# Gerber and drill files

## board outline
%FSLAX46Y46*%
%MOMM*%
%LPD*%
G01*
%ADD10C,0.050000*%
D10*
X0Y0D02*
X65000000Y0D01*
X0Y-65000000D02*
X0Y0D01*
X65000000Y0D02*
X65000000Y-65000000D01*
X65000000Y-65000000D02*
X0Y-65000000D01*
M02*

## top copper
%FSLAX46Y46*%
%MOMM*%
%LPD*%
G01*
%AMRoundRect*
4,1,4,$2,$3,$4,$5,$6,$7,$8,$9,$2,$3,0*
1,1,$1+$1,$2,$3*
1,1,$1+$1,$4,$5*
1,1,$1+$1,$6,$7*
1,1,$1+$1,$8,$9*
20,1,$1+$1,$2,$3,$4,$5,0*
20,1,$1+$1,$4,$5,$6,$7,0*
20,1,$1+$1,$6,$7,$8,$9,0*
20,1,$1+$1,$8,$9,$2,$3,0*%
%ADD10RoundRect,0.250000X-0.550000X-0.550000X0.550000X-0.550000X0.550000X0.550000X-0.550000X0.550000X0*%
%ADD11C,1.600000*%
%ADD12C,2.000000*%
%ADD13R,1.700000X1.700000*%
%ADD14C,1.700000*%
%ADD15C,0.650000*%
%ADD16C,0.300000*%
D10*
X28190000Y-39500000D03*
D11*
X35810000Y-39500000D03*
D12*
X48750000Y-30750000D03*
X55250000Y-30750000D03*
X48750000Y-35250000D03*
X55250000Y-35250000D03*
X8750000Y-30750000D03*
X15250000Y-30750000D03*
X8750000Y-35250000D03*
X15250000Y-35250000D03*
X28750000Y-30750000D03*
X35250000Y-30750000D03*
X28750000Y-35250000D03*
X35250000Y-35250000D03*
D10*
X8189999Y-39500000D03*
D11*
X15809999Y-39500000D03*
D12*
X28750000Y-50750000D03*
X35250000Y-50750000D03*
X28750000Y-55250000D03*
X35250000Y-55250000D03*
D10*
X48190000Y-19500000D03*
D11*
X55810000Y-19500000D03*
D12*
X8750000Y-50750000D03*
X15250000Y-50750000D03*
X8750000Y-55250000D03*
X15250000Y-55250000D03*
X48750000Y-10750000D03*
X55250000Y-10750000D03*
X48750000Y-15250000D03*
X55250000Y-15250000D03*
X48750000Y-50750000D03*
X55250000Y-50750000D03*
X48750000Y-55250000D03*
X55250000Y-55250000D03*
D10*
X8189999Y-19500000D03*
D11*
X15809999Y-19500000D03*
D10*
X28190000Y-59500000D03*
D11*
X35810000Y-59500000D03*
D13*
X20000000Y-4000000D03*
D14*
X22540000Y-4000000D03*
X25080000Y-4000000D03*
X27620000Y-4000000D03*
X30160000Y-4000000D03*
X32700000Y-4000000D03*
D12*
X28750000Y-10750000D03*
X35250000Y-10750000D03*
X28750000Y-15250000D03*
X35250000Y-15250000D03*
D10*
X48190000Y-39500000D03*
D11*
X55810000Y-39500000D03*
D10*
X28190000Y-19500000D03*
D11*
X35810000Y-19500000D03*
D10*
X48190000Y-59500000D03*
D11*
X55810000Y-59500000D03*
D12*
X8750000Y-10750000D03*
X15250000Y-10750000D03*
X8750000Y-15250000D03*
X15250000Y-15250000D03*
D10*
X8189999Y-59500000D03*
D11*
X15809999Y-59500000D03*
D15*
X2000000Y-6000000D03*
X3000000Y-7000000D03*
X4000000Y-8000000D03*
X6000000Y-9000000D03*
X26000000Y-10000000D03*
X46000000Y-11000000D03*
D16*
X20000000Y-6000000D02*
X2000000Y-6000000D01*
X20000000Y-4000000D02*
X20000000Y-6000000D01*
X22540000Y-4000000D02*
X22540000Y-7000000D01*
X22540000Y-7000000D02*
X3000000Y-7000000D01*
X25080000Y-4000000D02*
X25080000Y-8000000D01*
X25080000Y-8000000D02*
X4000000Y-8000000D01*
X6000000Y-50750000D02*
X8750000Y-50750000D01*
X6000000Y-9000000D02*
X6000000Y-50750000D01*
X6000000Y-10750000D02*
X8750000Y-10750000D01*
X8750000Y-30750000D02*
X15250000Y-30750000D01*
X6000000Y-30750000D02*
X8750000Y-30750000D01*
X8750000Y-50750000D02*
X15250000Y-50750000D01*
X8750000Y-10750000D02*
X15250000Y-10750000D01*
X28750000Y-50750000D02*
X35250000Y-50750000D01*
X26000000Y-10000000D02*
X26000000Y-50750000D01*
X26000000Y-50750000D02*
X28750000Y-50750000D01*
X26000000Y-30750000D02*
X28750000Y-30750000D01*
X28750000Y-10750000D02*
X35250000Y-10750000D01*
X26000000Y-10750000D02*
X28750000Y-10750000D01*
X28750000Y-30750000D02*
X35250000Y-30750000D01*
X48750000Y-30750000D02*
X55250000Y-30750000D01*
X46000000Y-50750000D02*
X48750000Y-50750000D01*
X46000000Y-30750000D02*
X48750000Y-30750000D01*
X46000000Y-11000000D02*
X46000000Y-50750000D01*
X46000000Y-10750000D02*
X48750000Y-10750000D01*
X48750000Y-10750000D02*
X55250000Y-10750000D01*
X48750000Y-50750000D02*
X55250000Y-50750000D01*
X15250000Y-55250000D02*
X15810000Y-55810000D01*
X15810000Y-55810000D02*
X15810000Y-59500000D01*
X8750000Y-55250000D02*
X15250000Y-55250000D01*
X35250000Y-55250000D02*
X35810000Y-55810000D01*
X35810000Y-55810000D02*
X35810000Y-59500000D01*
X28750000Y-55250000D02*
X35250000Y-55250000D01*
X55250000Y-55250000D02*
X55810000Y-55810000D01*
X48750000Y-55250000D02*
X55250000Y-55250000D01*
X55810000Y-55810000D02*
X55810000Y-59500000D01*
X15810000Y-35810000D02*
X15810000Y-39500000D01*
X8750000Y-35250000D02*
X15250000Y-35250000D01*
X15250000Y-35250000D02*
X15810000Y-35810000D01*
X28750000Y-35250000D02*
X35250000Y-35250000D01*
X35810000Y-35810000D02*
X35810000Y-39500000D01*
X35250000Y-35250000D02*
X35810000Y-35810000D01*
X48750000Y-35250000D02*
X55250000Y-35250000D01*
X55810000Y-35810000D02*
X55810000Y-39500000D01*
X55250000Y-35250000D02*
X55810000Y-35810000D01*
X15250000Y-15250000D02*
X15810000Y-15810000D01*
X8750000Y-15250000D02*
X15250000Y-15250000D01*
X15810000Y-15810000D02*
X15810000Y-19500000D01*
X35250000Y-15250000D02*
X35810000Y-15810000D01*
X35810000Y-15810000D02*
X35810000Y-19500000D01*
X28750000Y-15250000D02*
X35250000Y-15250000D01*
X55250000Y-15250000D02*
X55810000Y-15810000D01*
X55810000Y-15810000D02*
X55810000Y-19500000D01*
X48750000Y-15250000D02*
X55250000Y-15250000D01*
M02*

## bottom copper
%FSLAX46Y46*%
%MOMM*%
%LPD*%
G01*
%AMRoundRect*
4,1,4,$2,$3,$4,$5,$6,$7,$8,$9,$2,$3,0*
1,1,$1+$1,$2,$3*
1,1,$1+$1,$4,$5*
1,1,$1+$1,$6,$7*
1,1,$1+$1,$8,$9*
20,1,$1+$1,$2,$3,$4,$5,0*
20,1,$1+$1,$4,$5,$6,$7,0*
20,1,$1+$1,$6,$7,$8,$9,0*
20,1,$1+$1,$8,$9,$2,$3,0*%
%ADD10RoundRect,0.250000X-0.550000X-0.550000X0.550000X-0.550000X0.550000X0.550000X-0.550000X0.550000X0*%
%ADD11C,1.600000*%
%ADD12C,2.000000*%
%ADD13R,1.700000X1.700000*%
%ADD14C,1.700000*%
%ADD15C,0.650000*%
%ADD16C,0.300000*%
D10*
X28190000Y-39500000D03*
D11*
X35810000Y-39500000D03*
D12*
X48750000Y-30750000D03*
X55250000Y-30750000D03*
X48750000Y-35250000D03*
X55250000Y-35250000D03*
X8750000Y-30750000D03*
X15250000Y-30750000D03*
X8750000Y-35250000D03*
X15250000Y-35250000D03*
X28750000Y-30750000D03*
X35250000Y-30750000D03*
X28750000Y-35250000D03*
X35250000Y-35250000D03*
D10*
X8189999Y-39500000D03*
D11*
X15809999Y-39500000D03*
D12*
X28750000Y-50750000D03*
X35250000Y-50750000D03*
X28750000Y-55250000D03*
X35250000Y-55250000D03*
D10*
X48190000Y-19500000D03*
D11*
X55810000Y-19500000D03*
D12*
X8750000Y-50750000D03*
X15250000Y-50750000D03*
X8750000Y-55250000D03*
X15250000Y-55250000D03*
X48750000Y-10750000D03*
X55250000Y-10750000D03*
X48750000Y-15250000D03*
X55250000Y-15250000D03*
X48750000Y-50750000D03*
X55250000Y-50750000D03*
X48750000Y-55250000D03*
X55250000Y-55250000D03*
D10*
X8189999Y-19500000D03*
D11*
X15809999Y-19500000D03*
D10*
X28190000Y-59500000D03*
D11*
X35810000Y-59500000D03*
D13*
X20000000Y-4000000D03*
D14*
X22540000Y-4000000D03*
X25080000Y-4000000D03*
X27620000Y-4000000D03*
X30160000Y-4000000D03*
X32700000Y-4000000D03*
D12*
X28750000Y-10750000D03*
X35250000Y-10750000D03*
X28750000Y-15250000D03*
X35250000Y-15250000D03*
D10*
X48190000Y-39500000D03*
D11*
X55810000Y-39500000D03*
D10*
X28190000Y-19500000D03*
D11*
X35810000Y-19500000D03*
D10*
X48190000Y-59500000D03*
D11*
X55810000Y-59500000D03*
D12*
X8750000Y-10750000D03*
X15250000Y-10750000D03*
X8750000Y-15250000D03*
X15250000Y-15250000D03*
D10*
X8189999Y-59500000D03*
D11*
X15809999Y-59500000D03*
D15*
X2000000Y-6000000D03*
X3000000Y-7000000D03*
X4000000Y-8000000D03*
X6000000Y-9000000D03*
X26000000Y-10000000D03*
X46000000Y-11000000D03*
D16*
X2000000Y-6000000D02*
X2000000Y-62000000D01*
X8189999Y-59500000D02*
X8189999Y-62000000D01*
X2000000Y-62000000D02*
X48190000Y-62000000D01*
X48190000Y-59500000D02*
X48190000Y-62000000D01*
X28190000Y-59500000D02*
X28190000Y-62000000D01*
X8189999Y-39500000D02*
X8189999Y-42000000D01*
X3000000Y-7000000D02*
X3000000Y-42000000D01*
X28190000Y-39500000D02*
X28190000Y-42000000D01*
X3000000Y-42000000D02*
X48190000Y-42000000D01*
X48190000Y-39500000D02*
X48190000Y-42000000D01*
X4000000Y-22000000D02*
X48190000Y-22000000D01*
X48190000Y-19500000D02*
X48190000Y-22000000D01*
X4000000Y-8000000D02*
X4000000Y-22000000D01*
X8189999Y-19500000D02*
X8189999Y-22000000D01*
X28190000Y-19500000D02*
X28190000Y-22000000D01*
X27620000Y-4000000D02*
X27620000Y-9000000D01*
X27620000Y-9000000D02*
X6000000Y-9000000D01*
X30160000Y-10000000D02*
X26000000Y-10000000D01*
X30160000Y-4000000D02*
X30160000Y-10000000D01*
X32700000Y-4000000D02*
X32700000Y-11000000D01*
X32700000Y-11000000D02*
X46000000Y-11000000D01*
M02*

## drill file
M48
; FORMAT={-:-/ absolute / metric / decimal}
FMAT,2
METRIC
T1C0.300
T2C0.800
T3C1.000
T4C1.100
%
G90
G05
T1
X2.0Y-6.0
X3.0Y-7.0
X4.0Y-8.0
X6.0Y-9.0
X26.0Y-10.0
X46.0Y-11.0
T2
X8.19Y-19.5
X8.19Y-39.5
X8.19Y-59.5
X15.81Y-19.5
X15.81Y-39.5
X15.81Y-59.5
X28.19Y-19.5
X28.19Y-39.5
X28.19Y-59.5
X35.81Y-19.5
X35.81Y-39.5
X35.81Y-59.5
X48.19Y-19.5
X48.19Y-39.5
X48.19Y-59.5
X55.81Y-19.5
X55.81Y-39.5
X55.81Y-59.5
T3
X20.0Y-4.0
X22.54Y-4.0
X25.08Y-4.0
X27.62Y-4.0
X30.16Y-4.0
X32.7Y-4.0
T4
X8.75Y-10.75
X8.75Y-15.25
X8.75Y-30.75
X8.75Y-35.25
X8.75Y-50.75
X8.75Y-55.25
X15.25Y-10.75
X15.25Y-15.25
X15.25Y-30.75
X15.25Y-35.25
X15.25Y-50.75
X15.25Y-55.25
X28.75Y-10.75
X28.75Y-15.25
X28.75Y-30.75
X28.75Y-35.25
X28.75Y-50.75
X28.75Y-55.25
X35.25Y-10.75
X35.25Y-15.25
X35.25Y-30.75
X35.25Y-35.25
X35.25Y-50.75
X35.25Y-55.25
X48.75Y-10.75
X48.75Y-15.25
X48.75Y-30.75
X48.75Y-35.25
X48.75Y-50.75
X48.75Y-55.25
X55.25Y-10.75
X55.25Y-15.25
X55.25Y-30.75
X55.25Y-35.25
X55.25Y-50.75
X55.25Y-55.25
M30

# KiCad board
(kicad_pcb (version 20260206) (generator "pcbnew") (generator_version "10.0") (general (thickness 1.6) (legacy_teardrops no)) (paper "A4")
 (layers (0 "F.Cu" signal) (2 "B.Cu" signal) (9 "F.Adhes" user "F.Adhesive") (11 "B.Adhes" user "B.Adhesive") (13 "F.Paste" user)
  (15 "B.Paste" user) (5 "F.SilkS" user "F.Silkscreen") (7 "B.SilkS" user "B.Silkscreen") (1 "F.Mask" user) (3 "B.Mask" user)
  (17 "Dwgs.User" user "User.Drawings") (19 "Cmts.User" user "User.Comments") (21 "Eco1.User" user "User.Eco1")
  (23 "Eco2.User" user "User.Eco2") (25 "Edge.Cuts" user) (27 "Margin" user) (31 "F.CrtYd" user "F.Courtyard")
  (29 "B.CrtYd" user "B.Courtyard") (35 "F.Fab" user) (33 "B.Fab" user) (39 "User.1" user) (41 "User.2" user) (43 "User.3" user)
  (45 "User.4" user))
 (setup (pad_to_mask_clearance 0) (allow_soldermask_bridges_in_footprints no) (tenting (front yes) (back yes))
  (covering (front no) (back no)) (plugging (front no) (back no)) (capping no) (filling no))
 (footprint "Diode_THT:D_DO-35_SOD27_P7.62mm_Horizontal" (layer "F.Cu") (at 28.19 39.5)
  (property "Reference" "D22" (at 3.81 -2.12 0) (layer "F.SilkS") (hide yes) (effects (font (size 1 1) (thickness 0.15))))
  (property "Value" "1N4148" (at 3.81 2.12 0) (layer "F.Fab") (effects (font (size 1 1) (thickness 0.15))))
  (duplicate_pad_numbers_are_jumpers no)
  (pad "1" thru_hole roundrect (at 0 0) (size 1.6 1.6) (drill 0.8) (layers "*.Cu" "*.Mask") (remove_unused_layers no)
   (roundrect_rratio 0.15625) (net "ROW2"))
  (pad "2" thru_hole circle (at 7.62 0) (size 1.6 1.6) (drill 0.8) (layers "*.Cu" "*.Mask") (remove_unused_layers no) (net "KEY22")))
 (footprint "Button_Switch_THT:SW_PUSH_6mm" (layer "F.Cu") (at 48.75 30.75)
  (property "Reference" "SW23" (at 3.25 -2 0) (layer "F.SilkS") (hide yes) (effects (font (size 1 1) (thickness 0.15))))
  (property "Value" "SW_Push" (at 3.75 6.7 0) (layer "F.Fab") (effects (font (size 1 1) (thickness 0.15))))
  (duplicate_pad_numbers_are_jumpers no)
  (pad "1" thru_hole circle (at 0 0 90) (size 2 2) (drill 1.1) (layers "*.Cu" "*.Mask") (remove_unused_layers no) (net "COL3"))
  (pad "1" thru_hole circle (at 6.5 0 90) (size 2 2) (drill 1.1) (layers "*.Cu" "*.Mask") (remove_unused_layers no) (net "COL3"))
  (pad "2" thru_hole circle (at 0 4.5 90) (size 2 2) (drill 1.1) (layers "*.Cu" "*.Mask") (remove_unused_layers no) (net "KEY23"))
  (pad "2" thru_hole circle (at 6.5 4.5 90) (size 2 2) (drill 1.1) (layers "*.Cu" "*.Mask") (remove_unused_layers no) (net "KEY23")))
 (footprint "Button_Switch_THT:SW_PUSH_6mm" (layer "F.Cu") (at 8.75 30.75)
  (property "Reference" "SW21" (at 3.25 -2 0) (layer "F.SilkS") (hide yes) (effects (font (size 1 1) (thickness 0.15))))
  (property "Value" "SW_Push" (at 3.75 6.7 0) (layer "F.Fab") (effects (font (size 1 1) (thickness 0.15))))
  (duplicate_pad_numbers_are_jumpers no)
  (pad "1" thru_hole circle (at 0 0 90) (size 2 2) (drill 1.1) (layers "*.Cu" "*.Mask") (remove_unused_layers no) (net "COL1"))
  (pad "1" thru_hole circle (at 6.5 0 90) (size 2 2) (drill 1.1) (layers "*.Cu" "*.Mask") (remove_unused_layers no) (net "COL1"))
  (pad "2" thru_hole circle (at 0 4.5 90) (size 2 2) (drill 1.1) (layers "*.Cu" "*.Mask") (remove_unused_layers no) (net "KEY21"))
  (pad "2" thru_hole circle (at 6.5 4.5 90) (size 2 2) (drill 1.1) (layers "*.Cu" "*.Mask") (remove_unused_layers no) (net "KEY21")))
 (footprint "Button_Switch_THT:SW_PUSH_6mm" (layer "F.Cu") (at 28.75 30.75)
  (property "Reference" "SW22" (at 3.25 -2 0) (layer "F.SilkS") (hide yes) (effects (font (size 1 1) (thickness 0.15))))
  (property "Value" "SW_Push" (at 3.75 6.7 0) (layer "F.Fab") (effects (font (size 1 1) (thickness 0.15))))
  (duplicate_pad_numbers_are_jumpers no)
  (pad "1" thru_hole circle (at 0 0 90) (size 2 2) (drill 1.1) (layers "*.Cu" "*.Mask") (remove_unused_layers no) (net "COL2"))
  (pad "1" thru_hole circle (at 6.5 0 90) (size 2 2) (drill 1.1) (layers "*.Cu" "*.Mask") (remove_unused_layers no) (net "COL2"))
  (pad "2" thru_hole circle (at 0 4.5 90) (size 2 2) (drill 1.1) (layers "*.Cu" "*.Mask") (remove_unused_layers no) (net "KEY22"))
  (pad "2" thru_hole circle (at 6.5 4.5 90) (size 2 2) (drill 1.1) (layers "*.Cu" "*.Mask") (remove_unused_layers no) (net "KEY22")))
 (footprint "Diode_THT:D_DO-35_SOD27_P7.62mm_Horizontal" (layer "F.Cu") (at 8.189999 39.5)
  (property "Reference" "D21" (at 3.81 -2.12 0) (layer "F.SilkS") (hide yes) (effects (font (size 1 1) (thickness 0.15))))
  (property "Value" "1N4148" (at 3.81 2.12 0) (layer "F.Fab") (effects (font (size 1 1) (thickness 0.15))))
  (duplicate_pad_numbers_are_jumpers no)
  (pad "1" thru_hole roundrect (at 0 0) (size 1.6 1.6) (drill 0.8) (layers "*.Cu" "*.Mask") (remove_unused_layers no)
   (roundrect_rratio 0.15625) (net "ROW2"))
  (pad "2" thru_hole circle (at 7.62 0) (size 1.6 1.6) (drill 0.8) (layers "*.Cu" "*.Mask") (remove_unused_layers no) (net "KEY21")))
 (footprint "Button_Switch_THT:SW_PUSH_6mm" (layer "F.Cu") (at 28.75 50.75)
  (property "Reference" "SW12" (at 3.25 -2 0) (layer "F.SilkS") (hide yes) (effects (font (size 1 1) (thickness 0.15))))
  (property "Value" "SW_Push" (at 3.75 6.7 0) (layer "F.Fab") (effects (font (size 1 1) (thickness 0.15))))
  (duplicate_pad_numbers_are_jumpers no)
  (pad "1" thru_hole circle (at 0 0 90) (size 2 2) (drill 1.1) (layers "*.Cu" "*.Mask") (remove_unused_layers no) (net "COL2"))
  (pad "1" thru_hole circle (at 6.5 0 90) (size 2 2) (drill 1.1) (layers "*.Cu" "*.Mask") (remove_unused_layers no) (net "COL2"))
  (pad "2" thru_hole circle (at 0 4.5 90) (size 2 2) (drill 1.1) (layers "*.Cu" "*.Mask") (remove_unused_layers no) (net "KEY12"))
  (pad "2" thru_hole circle (at 6.5 4.5 90) (size 2 2) (drill 1.1) (layers "*.Cu" "*.Mask") (remove_unused_layers no) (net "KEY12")))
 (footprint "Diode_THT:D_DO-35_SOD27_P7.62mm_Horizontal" (layer "F.Cu") (at 48.19 19.5)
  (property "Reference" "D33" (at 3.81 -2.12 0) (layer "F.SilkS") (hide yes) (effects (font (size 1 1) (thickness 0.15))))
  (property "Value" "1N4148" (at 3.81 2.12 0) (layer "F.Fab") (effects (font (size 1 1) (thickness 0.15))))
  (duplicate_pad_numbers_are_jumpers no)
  (pad "1" thru_hole roundrect (at 0 0) (size 1.6 1.6) (drill 0.8) (layers "*.Cu" "*.Mask") (remove_unused_layers no)
   (roundrect_rratio 0.15625) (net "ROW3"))
  (pad "2" thru_hole circle (at 7.62 0) (size 1.6 1.6) (drill 0.8) (layers "*.Cu" "*.Mask") (remove_unused_layers no) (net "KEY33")))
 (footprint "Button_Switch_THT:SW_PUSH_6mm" (layer "F.Cu") (at 8.75 50.75)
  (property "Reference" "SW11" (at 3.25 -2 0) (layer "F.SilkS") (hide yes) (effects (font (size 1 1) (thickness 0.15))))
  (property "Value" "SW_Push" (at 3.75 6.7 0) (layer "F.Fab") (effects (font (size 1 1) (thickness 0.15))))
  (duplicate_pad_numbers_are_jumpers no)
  (pad "1" thru_hole circle (at 0 0 90) (size 2 2) (drill 1.1) (layers "*.Cu" "*.Mask") (remove_unused_layers no) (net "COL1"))
  (pad "1" thru_hole circle (at 6.5 0 90) (size 2 2) (drill 1.1) (layers "*.Cu" "*.Mask") (remove_unused_layers no) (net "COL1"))
  (pad "2" thru_hole circle (at 0 4.5 90) (size 2 2) (drill 1.1) (layers "*.Cu" "*.Mask") (remove_unused_layers no) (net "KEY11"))
  (pad "2" thru_hole circle (at 6.5 4.5 90) (size 2 2) (drill 1.1) (layers "*.Cu" "*.Mask") (remove_unused_layers no) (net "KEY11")))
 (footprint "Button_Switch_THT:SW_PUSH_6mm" (layer "F.Cu") (at 48.75 10.75)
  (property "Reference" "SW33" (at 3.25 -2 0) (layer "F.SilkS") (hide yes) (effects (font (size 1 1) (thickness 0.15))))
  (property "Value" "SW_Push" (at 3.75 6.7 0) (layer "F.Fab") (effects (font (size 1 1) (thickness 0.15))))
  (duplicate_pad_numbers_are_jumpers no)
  (pad "1" thru_hole circle (at 0 0 90) (size 2 2) (drill 1.1) (layers "*.Cu" "*.Mask") (remove_unused_layers no) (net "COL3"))
  (pad "1" thru_hole circle (at 6.5 0 90) (size 2 2) (drill 1.1) (layers "*.Cu" "*.Mask") (remove_unused_layers no) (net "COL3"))
  (pad "2" thru_hole circle (at 0 4.5 90) (size 2 2) (drill 1.1) (layers "*.Cu" "*.Mask") (remove_unused_layers no) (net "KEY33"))
  (pad "2" thru_hole circle (at 6.5 4.5 90) (size 2 2) (drill 1.1) (layers "*.Cu" "*.Mask") (remove_unused_layers no) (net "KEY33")))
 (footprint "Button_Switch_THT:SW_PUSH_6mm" (layer "F.Cu") (at 48.75 50.75)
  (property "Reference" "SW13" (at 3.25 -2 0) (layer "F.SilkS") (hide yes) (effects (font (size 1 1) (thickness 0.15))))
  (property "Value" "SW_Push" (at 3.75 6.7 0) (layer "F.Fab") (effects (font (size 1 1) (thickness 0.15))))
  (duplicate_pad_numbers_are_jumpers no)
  (pad "1" thru_hole circle (at 0 0 90) (size 2 2) (drill 1.1) (layers "*.Cu" "*.Mask") (remove_unused_layers no) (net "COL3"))
  (pad "1" thru_hole circle (at 6.5 0 90) (size 2 2) (drill 1.1) (layers "*.Cu" "*.Mask") (remove_unused_layers no) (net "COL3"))
  (pad "2" thru_hole circle (at 0 4.5 90) (size 2 2) (drill 1.1) (layers "*.Cu" "*.Mask") (remove_unused_layers no) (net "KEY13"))
  (pad "2" thru_hole circle (at 6.5 4.5 90) (size 2 2) (drill 1.1) (layers "*.Cu" "*.Mask") (remove_unused_layers no) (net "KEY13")))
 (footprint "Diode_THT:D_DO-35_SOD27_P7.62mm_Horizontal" (layer "F.Cu") (at 8.189999 19.5)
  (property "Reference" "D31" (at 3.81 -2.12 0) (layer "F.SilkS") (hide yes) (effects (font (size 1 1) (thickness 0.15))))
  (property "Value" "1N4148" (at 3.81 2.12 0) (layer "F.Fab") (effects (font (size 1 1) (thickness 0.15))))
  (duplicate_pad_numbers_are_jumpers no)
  (pad "1" thru_hole roundrect (at 0 0) (size 1.6 1.6) (drill 0.8) (layers "*.Cu" "*.Mask") (remove_unused_layers no)
   (roundrect_rratio 0.15625) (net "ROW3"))
  (pad "2" thru_hole circle (at 7.62 0) (size 1.6 1.6) (drill 0.8) (layers "*.Cu" "*.Mask") (remove_unused_layers no) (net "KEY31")))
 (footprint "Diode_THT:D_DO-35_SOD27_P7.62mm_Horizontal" (layer "F.Cu") (at 28.19 59.5)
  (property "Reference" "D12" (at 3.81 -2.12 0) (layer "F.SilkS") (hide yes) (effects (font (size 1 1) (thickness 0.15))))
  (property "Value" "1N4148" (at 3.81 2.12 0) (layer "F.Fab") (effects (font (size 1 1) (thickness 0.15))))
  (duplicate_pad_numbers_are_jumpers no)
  (pad "1" thru_hole roundrect (at 0 0) (size 1.6 1.6) (drill 0.8) (layers "*.Cu" "*.Mask") (remove_unused_layers no)
   (roundrect_rratio 0.15625) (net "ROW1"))
  (pad "2" thru_hole circle (at 7.62 0) (size 1.6 1.6) (drill 0.8) (layers "*.Cu" "*.Mask") (remove_unused_layers no) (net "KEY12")))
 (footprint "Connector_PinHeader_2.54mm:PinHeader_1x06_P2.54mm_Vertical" (layer "F.Cu") (at 20 4 90)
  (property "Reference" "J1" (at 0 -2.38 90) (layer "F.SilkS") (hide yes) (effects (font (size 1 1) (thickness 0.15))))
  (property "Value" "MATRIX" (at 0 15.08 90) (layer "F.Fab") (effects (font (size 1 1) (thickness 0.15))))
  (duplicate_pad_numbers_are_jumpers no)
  (pad "1" thru_hole rect (at 0 0 90) (size 1.7 1.7) (drill 1) (layers "*.Cu" "*.Mask") (remove_unused_layers no) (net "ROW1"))
  (pad "2" thru_hole circle (at 0 2.54 90) (size 1.7 1.7) (drill 1) (layers "*.Cu" "*.Mask") (remove_unused_layers no) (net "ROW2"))
  (pad "3" thru_hole circle (at 0 5.08 90) (size 1.7 1.7) (drill 1) (layers "*.Cu" "*.Mask") (remove_unused_layers no) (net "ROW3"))
  (pad "4" thru_hole circle (at 0 7.62 90) (size 1.7 1.7) (drill 1) (layers "*.Cu" "*.Mask") (remove_unused_layers no) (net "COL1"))
  (pad "5" thru_hole circle (at 0 10.16 90) (size 1.7 1.7) (drill 1) (layers "*.Cu" "*.Mask") (remove_unused_layers no) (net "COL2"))
  (pad "6" thru_hole circle (at 0 12.7 90) (size 1.7 1.7) (drill 1) (layers "*.Cu" "*.Mask") (remove_unused_layers no) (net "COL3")))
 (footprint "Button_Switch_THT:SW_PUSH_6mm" (layer "F.Cu") (at 28.75 10.75)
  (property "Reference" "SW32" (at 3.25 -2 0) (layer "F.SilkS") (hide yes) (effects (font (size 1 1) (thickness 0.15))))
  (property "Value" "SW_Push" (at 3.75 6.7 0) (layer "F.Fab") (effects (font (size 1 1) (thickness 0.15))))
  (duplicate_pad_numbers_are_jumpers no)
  (pad "1" thru_hole circle (at 0 0 90) (size 2 2) (drill 1.1) (layers "*.Cu" "*.Mask") (remove_unused_layers no) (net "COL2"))
  (pad "1" thru_hole circle (at 6.5 0 90) (size 2 2) (drill 1.1) (layers "*.Cu" "*.Mask") (remove_unused_layers no) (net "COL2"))
  (pad "2" thru_hole circle (at 0 4.5 90) (size 2 2) (drill 1.1) (layers "*.Cu" "*.Mask") (remove_unused_layers no) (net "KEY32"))
  (pad "2" thru_hole circle (at 6.5 4.5 90) (size 2 2) (drill 1.1) (layers "*.Cu" "*.Mask") (remove_unused_layers no) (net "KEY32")))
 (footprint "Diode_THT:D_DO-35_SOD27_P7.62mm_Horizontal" (layer "F.Cu") (at 48.19 39.5)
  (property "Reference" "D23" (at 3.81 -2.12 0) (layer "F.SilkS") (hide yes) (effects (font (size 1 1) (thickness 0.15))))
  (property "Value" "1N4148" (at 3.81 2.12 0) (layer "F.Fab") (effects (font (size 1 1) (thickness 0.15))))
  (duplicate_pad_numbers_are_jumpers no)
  (pad "1" thru_hole roundrect (at 0 0) (size 1.6 1.6) (drill 0.8) (layers "*.Cu" "*.Mask") (remove_unused_layers no)
   (roundrect_rratio 0.15625) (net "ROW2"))
  (pad "2" thru_hole circle (at 7.62 0) (size 1.6 1.6) (drill 0.8) (layers "*.Cu" "*.Mask") (remove_unused_layers no) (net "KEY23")))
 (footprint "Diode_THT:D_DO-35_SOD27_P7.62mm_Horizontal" (layer "F.Cu") (at 28.19 19.5)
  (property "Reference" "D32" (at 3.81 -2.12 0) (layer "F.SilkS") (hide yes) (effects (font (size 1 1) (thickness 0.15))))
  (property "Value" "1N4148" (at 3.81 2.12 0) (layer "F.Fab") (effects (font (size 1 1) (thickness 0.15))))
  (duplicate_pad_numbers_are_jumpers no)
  (pad "1" thru_hole roundrect (at 0 0) (size 1.6 1.6) (drill 0.8) (layers "*.Cu" "*.Mask") (remove_unused_layers no)
   (roundrect_rratio 0.15625) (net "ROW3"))
  (pad "2" thru_hole circle (at 7.62 0) (size 1.6 1.6) (drill 0.8) (layers "*.Cu" "*.Mask") (remove_unused_layers no) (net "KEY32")))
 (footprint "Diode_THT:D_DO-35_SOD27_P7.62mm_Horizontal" (layer "F.Cu") (at 48.19 59.5)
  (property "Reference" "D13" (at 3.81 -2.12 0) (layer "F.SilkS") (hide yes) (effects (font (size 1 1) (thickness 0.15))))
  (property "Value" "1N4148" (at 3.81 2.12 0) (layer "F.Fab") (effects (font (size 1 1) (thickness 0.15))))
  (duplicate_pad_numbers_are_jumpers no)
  (pad "1" thru_hole roundrect (at 0 0) (size 1.6 1.6) (drill 0.8) (layers "*.Cu" "*.Mask") (remove_unused_layers no)
   (roundrect_rratio 0.15625) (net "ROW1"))
  (pad "2" thru_hole circle (at 7.62 0) (size 1.6 1.6) (drill 0.8) (layers "*.Cu" "*.Mask") (remove_unused_layers no) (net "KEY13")))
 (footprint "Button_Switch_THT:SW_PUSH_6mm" (layer "F.Cu") (at 8.75 10.75)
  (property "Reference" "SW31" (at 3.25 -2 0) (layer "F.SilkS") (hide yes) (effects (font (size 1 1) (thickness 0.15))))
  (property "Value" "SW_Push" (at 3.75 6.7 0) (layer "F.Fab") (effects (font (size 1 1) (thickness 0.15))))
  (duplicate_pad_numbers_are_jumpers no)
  (pad "1" thru_hole circle (at 0 0 90) (size 2 2) (drill 1.1) (layers "*.Cu" "*.Mask") (remove_unused_layers no) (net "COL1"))
  (pad "1" thru_hole circle (at 6.5 0 90) (size 2 2) (drill 1.1) (layers "*.Cu" "*.Mask") (remove_unused_layers no) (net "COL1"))
  (pad "2" thru_hole circle (at 0 4.5 90) (size 2 2) (drill 1.1) (layers "*.Cu" "*.Mask") (remove_unused_layers no) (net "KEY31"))
  (pad "2" thru_hole circle (at 6.5 4.5 90) (size 2 2) (drill 1.1) (layers "*.Cu" "*.Mask") (remove_unused_layers no) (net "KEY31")))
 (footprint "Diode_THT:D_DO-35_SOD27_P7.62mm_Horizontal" (layer "F.Cu") (at 8.189999 59.5)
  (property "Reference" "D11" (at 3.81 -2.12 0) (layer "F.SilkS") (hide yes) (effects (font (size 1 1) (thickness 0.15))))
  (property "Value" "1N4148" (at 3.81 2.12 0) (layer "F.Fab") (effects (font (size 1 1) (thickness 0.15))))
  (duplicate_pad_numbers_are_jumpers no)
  (pad "1" thru_hole roundrect (at 0 0) (size 1.6 1.6) (drill 0.8) (layers "*.Cu" "*.Mask") (remove_unused_layers no)
   (roundrect_rratio 0.15625) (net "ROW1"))
  (pad "2" thru_hole circle (at 7.62 0) (size 1.6 1.6) (drill 0.8) (layers "*.Cu" "*.Mask") (remove_unused_layers no) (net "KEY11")))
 (gr_line (start 0 0) (end 65 0) (stroke (width 0.05) (type default)) (layer "Edge.Cuts"))
 (gr_line (start 0 65) (end 0 0) (stroke (width 0.05) (type default)) (layer "Edge.Cuts"))
 (gr_line (start 65 0) (end 65 65) (stroke (width 0.05) (type default)) (layer "Edge.Cuts"))
 (gr_line (start 65 65) (end 0 65) (stroke (width 0.05) (type default)) (layer "Edge.Cuts"))
 (segment (start 20 6) (end 2 6) (width 0.3) (layer "F.Cu") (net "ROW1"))
 (segment (start 20 4) (end 20 6) (width 0.3) (layer "F.Cu") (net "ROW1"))
 (via (at 2 6) (size 0.65) (drill 0.3) (layers "F.Cu" "B.Cu") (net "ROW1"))
 (segment (start 2 6) (end 2 62) (width 0.3) (layer "B.Cu") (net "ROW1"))
 (segment (start 8.189999 59.5) (end 8.189999 62) (width 0.3) (layer "B.Cu") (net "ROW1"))
 (segment (start 2 62) (end 48.19 62) (width 0.3) (layer "B.Cu") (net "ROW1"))
 (segment (start 48.19 59.5) (end 48.19 62) (width 0.3) (layer "B.Cu") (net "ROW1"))
 (segment (start 28.19 59.5) (end 28.19 62) (width 0.3) (layer "B.Cu") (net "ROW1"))
 (segment (start 22.54 4) (end 22.54 7) (width 0.3) (layer "F.Cu") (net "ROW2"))
 (segment (start 22.54 7) (end 3 7) (width 0.3) (layer "F.Cu") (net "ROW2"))
 (via (at 3 7) (size 0.65) (drill 0.3) (layers "F.Cu" "B.Cu") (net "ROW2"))
 (segment (start 8.189999 39.5) (end 8.189999 42) (width 0.3) (layer "B.Cu") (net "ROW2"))
 (segment (start 3 7) (end 3 42) (width 0.3) (layer "B.Cu") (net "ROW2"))
 (segment (start 28.19 39.5) (end 28.19 42) (width 0.3) (layer "B.Cu") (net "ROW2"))
 (segment (start 3 42) (end 48.19 42) (width 0.3) (layer "B.Cu") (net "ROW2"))
 (segment (start 48.19 39.5) (end 48.19 42) (width 0.3) (layer "B.Cu") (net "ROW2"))
 (segment (start 25.08 4) (end 25.08 8) (width 0.3) (layer "F.Cu") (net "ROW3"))
 (segment (start 25.08 8) (end 4 8) (width 0.3) (layer "F.Cu") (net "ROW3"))
 (via (at 4 8) (size 0.65) (drill 0.3) (layers "F.Cu" "B.Cu") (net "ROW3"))
 (segment (start 4 22) (end 48.19 22) (width 0.3) (layer "B.Cu") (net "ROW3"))
 (segment (start 48.19 19.5) (end 48.19 22) (width 0.3) (layer "B.Cu") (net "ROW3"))
 (segment (start 4 8) (end 4 22) (width 0.3) (layer "B.Cu") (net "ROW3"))
 (segment (start 8.189999 19.5) (end 8.189999 22) (width 0.3) (layer "B.Cu") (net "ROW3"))
 (segment (start 28.19 19.5) (end 28.19 22) (width 0.3) (layer "B.Cu") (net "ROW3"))
 (segment (start 6 50.75) (end 8.75 50.75) (width 0.3) (layer "F.Cu") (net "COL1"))
 (segment (start 6 9) (end 6 50.75) (width 0.3) (layer "F.Cu") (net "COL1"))
 (segment (start 6 10.75) (end 8.75 10.75) (width 0.3) (layer "F.Cu") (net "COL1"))
 (segment (start 8.75 30.75) (end 15.25 30.75) (width 0.3) (layer "F.Cu") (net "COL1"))
 (segment (start 6 30.75) (end 8.75 30.75) (width 0.3) (layer "F.Cu") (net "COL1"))
 (segment (start 8.75 50.75) (end 15.25 50.75) (width 0.3) (layer "F.Cu") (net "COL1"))
 (segment (start 8.75 10.75) (end 15.25 10.75) (width 0.3) (layer "F.Cu") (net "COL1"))
 (via (at 6 9) (size 0.65) (drill 0.3) (layers "F.Cu" "B.Cu") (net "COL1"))
 (segment (start 27.62 4) (end 27.62 9) (width 0.3) (layer "B.Cu") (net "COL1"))
 (segment (start 27.62 9) (end 6 9) (width 0.3) (layer "B.Cu") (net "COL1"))
 (segment (start 28.75 50.75) (end 35.25 50.75) (width 0.3) (layer "F.Cu") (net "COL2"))
 (segment (start 26 10) (end 26 50.75) (width 0.3) (layer "F.Cu") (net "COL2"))
 (segment (start 26 50.75) (end 28.75 50.75) (width 0.3) (layer "F.Cu") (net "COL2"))
 (segment (start 26 30.75) (end 28.75 30.75) (width 0.3) (layer "F.Cu") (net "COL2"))
 (segment (start 28.75 10.75) (end 35.25 10.75) (width 0.3) (layer "F.Cu") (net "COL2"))
 (segment (start 26 10.75) (end 28.75 10.75) (width 0.3) (layer "F.Cu") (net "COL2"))
 (segment (start 28.75 30.75) (end 35.25 30.75) (width 0.3) (layer "F.Cu") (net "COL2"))
 (via (at 26 10) (size 0.65) (drill 0.3) (layers "F.Cu" "B.Cu") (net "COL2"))
 (segment (start 30.16 10) (end 26 10) (width 0.3) (layer "B.Cu") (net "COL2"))
 (segment (start 30.16 4) (end 30.16 10) (width 0.3) (layer "B.Cu") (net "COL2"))
 (segment (start 48.75 30.75) (end 55.25 30.75) (width 0.3) (layer "F.Cu") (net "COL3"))
 (segment (start 46 50.75) (end 48.75 50.75) (width 0.3) (layer "F.Cu") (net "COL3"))
 (segment (start 46 30.75) (end 48.75 30.75) (width 0.3) (layer "F.Cu") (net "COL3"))
 (segment (start 46 11) (end 46 50.75) (width 0.3) (layer "F.Cu") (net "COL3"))
 (segment (start 46 10.75) (end 48.75 10.75) (width 0.3) (layer "F.Cu") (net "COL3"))
 (segment (start 48.75 10.75) (end 55.25 10.75) (width 0.3) (layer "F.Cu") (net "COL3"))
 (segment (start 48.75 50.75) (end 55.25 50.75) (width 0.3) (layer "F.Cu") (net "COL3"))
 (via (at 46 11) (size 0.65) (drill 0.3) (layers "F.Cu" "B.Cu") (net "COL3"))
 (segment (start 32.7 4) (end 32.7 11) (width 0.3) (layer "B.Cu") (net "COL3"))
 (segment (start 32.7 11) (end 46 11) (width 0.3) (layer "B.Cu") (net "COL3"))
 (segment (start 15.25 55.25) (end 15.81 55.81) (width 0.3) (layer "F.Cu") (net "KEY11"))
 (segment (start 15.81 55.81) (end 15.81 59.5) (width 0.3) (layer "F.Cu") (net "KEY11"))
 (segment (start 8.75 55.25) (end 15.25 55.25) (width 0.3) (layer "F.Cu") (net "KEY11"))
 (segment (start 35.25 55.25) (end 35.81 55.81) (width 0.3) (layer "F.Cu") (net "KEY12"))
 (segment (start 35.81 55.81) (end 35.81 59.5) (width 0.3) (layer "F.Cu") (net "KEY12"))
 (segment (start 28.75 55.25) (end 35.25 55.25) (width 0.3) (layer "F.Cu") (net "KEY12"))
 (segment (start 55.25 55.25) (end 55.81 55.81) (width 0.3) (layer "F.Cu") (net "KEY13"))
 (segment (start 48.75 55.25) (end 55.25 55.25) (width 0.3) (layer "F.Cu") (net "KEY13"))
 (segment (start 55.81 55.81) (end 55.81 59.5) (width 0.3) (layer "F.Cu") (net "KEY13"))
 (segment (start 15.81 35.81) (end 15.81 39.5) (width 0.3) (layer "F.Cu") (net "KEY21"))
 (segment (start 8.75 35.25) (end 15.25 35.25) (width 0.3) (layer "F.Cu") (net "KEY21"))
 (segment (start 15.25 35.25) (end 15.81 35.81) (width 0.3) (layer "F.Cu") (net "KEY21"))
 (segment (start 28.75 35.25) (end 35.25 35.25) (width 0.3) (layer "F.Cu") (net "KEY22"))
 (segment (start 35.81 35.81) (end 35.81 39.5) (width 0.3) (layer "F.Cu") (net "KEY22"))
 (segment (start 35.25 35.25) (end 35.81 35.81) (width 0.3) (layer "F.Cu") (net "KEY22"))
 (segment (start 48.75 35.25) (end 55.25 35.25) (width 0.3) (layer "F.Cu") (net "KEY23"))
 (segment (start 55.81 35.81) (end 55.81 39.5) (width 0.3) (layer "F.Cu") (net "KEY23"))
 (segment (start 55.25 35.25) (end 55.81 35.81) (width 0.3) (layer "F.Cu") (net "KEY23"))
 (segment (start 15.25 15.25) (end 15.81 15.81) (width 0.3) (layer "F.Cu") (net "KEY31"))
 (segment (start 8.75 15.25) (end 15.25 15.25) (width 0.3) (layer "F.Cu") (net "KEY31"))
 (segment (start 15.81 15.81) (end 15.81 19.5) (width 0.3) (layer "F.Cu") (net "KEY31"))
 (segment (start 35.25 15.25) (end 35.81 15.81) (width 0.3) (layer "F.Cu") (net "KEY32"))
 (segment (start 35.81 15.81) (end 35.81 19.5) (width 0.3) (layer "F.Cu") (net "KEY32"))
 (segment (start 28.75 15.25) (end 35.25 15.25) (width 0.3) (layer "F.Cu") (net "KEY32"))
 (segment (start 55.25 15.25) (end 55.81 15.81) (width 0.3) (layer "F.Cu") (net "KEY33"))
 (segment (start 55.81 15.81) (end 55.81 19.5) (width 0.3) (layer "F.Cu") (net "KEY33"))
 (segment (start 48.75 15.25) (end 55.25 15.25) (width 0.3) (layer "F.Cu") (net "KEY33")))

